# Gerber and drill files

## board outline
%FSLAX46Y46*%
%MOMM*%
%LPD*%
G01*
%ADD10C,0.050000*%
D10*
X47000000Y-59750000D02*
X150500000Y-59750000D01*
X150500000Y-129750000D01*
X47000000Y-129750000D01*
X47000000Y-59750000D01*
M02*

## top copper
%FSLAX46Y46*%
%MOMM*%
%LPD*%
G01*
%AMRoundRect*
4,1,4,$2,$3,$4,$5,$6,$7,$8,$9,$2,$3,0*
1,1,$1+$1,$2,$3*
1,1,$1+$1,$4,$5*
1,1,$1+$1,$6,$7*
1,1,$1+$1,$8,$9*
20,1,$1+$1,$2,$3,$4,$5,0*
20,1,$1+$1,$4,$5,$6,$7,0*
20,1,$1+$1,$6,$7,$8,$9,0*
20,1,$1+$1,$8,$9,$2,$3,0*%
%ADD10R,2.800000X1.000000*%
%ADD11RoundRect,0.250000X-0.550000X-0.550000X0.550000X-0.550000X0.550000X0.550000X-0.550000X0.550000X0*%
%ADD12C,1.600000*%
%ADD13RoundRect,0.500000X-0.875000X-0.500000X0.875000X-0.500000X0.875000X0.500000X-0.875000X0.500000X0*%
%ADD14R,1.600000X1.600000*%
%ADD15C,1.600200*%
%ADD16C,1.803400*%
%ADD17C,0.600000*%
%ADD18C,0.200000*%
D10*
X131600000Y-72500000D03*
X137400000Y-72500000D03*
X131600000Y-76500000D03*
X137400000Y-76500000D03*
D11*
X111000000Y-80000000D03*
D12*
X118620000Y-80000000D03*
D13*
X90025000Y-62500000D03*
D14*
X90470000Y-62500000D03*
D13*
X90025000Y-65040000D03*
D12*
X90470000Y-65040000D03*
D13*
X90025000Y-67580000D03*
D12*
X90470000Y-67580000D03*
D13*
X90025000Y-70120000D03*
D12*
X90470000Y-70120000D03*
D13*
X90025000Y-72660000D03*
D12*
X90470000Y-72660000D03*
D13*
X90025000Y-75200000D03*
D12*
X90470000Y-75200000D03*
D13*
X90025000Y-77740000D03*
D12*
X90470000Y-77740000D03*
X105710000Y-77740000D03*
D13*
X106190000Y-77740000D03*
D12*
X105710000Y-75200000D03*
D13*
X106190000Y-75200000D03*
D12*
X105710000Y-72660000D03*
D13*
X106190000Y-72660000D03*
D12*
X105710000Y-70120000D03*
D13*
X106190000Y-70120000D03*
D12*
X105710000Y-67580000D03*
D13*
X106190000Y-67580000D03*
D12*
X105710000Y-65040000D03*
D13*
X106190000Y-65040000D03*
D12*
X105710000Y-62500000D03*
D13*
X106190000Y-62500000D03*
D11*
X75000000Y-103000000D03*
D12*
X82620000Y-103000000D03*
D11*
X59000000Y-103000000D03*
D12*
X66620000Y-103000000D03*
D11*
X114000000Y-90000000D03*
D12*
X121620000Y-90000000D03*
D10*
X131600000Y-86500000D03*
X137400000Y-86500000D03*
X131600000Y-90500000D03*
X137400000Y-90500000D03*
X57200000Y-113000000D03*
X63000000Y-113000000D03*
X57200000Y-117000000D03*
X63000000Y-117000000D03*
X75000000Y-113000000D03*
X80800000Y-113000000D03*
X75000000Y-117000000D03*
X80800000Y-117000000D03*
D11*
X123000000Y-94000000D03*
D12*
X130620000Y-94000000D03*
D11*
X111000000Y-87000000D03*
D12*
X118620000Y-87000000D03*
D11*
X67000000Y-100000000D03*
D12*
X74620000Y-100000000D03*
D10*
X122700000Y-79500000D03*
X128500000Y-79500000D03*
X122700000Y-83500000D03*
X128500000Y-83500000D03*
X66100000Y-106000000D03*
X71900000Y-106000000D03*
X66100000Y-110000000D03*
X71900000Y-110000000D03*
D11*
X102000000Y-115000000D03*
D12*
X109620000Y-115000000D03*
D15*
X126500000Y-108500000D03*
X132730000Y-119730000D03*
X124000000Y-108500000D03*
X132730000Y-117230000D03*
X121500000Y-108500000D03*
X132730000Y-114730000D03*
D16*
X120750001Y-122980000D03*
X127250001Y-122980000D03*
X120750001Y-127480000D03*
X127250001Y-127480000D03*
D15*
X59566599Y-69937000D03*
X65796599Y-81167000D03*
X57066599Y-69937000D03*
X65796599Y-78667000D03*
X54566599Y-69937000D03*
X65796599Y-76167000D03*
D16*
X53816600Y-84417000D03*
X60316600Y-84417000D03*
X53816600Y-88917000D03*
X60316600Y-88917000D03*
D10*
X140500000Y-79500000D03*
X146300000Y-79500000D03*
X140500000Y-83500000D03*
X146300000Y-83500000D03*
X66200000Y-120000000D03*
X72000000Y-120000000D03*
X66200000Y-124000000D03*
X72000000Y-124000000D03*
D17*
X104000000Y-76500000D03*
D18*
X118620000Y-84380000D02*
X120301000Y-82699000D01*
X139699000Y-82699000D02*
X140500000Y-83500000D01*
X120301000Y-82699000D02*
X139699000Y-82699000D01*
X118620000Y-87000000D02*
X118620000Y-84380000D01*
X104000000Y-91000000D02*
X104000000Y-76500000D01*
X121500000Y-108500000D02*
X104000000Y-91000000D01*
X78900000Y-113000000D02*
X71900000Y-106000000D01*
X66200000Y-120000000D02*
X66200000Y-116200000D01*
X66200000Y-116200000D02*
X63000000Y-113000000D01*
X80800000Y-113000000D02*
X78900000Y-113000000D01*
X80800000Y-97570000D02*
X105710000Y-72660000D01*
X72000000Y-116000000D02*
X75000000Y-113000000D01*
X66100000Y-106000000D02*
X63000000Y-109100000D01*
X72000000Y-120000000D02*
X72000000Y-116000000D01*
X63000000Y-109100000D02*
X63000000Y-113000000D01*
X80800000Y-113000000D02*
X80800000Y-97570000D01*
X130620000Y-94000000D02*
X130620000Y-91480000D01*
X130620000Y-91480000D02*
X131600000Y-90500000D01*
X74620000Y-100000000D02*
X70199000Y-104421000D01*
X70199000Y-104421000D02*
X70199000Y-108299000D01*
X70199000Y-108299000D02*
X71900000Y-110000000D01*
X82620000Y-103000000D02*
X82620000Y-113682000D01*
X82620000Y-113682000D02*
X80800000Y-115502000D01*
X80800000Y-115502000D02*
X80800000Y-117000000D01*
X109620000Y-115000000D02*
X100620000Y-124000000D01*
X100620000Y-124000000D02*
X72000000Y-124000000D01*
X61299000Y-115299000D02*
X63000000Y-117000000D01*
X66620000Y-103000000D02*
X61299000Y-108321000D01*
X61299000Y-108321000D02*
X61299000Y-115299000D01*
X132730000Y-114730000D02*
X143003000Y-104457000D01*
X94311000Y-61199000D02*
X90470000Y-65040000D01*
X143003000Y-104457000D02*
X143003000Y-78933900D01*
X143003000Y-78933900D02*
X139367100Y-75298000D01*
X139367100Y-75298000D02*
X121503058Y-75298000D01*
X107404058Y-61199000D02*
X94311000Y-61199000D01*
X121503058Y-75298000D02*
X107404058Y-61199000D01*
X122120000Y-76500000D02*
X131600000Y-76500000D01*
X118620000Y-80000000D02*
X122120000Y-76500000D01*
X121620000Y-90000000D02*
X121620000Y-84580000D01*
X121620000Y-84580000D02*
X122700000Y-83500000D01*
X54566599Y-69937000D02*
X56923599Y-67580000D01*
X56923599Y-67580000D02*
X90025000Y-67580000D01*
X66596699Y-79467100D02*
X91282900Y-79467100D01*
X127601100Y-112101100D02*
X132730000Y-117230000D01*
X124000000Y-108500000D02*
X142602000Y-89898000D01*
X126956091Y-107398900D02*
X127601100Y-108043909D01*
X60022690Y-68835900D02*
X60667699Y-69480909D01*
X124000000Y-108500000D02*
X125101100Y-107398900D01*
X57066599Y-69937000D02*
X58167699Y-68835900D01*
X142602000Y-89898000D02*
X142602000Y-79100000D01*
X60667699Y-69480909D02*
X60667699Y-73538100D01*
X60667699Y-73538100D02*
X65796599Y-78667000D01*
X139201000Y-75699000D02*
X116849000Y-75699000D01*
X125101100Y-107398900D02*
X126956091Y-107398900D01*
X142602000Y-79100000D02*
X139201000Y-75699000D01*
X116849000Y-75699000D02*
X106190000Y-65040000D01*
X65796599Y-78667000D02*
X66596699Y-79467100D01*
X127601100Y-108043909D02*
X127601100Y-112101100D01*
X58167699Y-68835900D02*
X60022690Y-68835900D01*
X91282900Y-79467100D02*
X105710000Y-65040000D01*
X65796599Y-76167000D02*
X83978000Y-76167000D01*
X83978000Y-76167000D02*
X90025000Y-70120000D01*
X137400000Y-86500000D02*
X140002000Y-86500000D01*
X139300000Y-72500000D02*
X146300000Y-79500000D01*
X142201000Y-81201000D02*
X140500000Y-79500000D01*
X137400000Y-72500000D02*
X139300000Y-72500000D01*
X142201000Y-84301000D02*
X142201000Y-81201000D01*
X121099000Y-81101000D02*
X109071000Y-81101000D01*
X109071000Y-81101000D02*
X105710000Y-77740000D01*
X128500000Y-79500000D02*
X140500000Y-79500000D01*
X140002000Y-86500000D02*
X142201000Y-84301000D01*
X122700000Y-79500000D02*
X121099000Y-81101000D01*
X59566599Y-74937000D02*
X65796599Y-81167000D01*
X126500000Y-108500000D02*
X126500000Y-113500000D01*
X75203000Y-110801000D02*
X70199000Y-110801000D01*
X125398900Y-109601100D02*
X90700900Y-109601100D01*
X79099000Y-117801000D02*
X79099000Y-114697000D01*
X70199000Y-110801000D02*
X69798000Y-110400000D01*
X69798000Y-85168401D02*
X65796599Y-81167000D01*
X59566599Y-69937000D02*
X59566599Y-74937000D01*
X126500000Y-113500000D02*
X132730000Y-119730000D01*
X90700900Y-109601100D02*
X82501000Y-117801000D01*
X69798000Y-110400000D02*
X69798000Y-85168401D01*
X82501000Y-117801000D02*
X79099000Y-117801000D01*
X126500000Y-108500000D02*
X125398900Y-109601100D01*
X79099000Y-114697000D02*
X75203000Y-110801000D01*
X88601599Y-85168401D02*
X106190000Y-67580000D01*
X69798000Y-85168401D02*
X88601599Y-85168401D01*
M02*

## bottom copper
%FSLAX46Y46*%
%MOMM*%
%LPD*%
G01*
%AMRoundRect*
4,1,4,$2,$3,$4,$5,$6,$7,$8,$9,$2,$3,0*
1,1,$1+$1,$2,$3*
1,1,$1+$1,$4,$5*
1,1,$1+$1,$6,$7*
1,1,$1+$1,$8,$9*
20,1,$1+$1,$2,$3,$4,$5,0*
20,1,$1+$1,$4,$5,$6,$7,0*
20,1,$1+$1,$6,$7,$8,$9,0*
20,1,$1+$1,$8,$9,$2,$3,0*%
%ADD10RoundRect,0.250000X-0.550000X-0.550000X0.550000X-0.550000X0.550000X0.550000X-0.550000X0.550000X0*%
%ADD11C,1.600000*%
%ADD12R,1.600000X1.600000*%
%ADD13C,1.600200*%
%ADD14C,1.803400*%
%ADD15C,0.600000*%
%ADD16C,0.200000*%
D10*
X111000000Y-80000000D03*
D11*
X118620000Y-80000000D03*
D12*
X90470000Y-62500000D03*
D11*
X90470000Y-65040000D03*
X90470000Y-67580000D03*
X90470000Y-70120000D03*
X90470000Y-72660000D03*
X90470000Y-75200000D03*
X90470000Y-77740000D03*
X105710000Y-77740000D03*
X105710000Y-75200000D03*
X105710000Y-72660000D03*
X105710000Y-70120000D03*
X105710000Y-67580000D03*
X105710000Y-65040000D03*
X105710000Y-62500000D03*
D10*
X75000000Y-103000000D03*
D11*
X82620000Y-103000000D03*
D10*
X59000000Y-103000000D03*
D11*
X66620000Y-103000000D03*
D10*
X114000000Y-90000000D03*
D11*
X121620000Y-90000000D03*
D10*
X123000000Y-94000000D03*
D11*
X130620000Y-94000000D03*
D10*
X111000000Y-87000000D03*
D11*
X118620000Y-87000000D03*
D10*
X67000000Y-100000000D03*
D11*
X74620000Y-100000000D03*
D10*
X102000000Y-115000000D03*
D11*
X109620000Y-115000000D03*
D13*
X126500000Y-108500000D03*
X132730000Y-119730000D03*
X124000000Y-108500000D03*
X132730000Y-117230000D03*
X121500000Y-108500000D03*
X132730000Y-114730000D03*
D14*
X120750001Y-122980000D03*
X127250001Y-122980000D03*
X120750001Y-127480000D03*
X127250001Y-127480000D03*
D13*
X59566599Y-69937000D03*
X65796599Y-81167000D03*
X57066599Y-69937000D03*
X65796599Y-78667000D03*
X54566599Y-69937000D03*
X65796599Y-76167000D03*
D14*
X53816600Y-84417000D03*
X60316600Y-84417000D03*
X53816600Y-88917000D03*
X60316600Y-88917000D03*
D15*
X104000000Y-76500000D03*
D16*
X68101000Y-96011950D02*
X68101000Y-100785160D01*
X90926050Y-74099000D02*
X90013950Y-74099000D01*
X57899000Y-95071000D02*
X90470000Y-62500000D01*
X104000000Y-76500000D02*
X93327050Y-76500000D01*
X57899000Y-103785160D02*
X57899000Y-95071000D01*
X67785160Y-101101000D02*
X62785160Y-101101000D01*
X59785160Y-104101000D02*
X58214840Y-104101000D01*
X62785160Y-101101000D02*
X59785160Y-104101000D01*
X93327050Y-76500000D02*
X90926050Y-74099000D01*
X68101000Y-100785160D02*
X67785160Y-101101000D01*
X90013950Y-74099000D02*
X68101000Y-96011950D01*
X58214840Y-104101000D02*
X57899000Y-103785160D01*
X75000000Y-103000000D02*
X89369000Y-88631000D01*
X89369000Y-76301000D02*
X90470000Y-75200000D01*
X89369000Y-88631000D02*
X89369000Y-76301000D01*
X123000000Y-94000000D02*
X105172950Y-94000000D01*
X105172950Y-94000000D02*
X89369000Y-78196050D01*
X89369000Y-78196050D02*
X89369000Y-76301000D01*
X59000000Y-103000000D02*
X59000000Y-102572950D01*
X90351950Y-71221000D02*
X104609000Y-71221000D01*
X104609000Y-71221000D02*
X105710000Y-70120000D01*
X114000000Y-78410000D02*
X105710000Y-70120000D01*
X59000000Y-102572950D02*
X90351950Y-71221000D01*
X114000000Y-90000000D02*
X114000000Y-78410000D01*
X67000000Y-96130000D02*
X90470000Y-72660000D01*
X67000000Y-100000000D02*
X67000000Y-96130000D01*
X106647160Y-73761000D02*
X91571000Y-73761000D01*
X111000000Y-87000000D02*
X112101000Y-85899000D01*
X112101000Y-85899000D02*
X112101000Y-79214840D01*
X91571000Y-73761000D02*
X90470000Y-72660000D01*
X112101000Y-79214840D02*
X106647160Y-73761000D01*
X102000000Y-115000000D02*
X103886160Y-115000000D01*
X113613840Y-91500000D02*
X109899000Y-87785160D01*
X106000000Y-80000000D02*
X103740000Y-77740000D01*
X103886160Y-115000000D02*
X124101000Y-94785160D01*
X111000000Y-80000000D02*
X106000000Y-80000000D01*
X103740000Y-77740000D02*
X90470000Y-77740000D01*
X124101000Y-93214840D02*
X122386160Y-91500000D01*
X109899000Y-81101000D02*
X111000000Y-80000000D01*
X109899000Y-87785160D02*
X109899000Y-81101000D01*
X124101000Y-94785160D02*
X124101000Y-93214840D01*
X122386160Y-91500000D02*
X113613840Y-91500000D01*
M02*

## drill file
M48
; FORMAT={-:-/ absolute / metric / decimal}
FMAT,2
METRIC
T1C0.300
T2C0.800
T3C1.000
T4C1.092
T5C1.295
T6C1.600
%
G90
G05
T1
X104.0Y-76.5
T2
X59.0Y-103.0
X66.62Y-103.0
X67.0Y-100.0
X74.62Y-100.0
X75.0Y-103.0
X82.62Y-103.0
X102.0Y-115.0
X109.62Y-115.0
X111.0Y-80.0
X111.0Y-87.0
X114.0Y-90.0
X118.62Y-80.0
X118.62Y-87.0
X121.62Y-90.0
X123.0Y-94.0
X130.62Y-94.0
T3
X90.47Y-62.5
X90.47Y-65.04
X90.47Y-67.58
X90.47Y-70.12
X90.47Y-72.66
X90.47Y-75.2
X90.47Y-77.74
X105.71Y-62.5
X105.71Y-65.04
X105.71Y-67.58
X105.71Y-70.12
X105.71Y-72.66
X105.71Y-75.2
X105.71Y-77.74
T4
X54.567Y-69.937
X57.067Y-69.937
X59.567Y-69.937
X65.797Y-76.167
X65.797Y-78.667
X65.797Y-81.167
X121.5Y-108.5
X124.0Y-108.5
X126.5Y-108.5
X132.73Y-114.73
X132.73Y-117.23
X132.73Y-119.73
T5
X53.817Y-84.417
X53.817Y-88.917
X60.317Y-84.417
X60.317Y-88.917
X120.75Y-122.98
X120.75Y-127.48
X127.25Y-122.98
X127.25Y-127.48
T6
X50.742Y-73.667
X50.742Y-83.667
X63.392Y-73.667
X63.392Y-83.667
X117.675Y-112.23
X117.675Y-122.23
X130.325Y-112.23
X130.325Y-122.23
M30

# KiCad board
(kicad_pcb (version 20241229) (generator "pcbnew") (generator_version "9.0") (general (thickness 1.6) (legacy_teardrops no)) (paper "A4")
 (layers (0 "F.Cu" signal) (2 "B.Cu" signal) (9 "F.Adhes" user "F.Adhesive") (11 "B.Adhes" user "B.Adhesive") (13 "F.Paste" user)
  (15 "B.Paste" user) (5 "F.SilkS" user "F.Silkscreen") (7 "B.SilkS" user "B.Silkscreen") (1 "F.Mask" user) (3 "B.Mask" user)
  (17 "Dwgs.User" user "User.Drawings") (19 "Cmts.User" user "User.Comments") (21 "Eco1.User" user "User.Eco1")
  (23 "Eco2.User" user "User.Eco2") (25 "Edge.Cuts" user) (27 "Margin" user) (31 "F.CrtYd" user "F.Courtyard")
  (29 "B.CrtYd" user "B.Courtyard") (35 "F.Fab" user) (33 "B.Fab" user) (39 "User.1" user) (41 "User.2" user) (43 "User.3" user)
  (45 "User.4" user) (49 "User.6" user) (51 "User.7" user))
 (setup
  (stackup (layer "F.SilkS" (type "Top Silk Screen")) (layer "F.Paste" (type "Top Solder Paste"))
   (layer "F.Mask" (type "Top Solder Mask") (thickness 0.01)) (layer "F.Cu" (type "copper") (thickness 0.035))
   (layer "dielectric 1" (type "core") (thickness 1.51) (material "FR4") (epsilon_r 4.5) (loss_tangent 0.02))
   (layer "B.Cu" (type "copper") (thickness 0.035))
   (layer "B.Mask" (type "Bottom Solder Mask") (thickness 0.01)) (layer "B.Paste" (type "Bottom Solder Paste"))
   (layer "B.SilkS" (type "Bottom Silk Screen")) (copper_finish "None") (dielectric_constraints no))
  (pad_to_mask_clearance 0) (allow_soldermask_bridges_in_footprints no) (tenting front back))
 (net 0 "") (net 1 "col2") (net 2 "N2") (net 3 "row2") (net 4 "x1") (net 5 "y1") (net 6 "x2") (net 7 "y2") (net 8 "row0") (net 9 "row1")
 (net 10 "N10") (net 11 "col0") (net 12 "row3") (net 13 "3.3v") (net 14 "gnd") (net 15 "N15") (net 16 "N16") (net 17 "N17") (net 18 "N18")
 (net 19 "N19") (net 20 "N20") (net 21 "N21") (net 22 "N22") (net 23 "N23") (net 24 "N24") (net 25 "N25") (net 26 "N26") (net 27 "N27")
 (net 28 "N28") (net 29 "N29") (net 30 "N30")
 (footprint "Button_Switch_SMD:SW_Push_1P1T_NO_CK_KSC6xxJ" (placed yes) (layer "F.Cu") (at 134.5 74.5)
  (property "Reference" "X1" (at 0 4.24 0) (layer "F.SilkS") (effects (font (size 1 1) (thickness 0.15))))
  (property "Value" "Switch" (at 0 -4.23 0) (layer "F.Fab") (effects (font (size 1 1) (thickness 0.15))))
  (pad "1" smd rect (at -2.9 -2) (size 2.8 1) (layers "F.Cu" "F.Mask" "F.Paste") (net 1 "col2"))
  (pad "1" smd rect (at 2.9 -2) (size 2.8 1) (layers "F.Cu" "F.Mask" "F.Paste") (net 1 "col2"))
  (pad "2" smd rect (at -2.9 2) (size 2.8 1) (layers "F.Cu" "F.Mask" "F.Paste") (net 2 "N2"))
  (pad "2" smd rect (at 2.9 2) (size 2.8 1) (layers "F.Cu" "F.Mask" "F.Paste") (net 2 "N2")))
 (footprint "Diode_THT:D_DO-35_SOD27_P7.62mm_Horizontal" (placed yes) (layer "F.Cu") (at 111 80)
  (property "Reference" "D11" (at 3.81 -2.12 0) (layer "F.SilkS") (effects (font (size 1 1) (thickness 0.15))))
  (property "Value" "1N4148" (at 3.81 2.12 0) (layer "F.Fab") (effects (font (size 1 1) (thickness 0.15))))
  (pad "1" thru_hole roundrect (at 0 0) (size 1.6 1.6) (drill 0.8) (layers "*.Cu" "*.Mask") (remove_unused_layers no)
   (roundrect_rratio 0.15625) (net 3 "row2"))
  (pad "2" thru_hole circle (at 7.62 0) (size 1.6 1.6) (drill 0.8) (layers "*.Cu" "*.Mask") (remove_unused_layers no) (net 2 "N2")))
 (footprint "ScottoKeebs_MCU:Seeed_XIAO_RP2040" (layer "F.Cu") (at 98.09 70.12)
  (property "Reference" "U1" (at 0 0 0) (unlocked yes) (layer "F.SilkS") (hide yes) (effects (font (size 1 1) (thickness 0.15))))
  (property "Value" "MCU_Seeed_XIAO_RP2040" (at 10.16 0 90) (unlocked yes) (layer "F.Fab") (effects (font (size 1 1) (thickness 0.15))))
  (pad "1" smd roundrect (at -8.065 -7.62) (size 2.75 2) (layers "F.Cu" "F.Mask" "F.Paste") (roundrect_rratio 0.25) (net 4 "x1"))
  (pad "1" thru_hole rect (at -7.62 -7.62 90) (size 1.6 1.6) (drill 1) (layers "*.Cu" "*.Mask") (remove_unused_layers no) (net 4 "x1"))
  (pad "2" smd roundrect (at -8.065 -5.08) (size 2.75 2) (layers "F.Cu" "F.Mask" "F.Paste") (roundrect_rratio 0.25) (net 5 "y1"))
  (pad "2" thru_hole circle (at -7.62 -5.08 90) (size 1.6 1.6) (drill 1) (layers "*.Cu" "*.Mask") (remove_unused_layers no) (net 5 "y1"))
  (pad "3" smd roundrect (at -8.065 -2.54) (size 2.75 2) (layers "F.Cu" "F.Mask" "F.Paste") (roundrect_rratio 0.25) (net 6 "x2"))
  (pad "3" thru_hole circle (at -7.62 -2.54 90) (size 1.6 1.6) (drill 1) (layers "*.Cu" "*.Mask") (remove_unused_layers no) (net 6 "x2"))
  (pad "4" smd roundrect (at -8.065 0) (size 2.75 2) (layers "F.Cu" "F.Mask" "F.Paste") (roundrect_rratio 0.25) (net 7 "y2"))
  (pad "4" thru_hole circle (at -7.62 0 90) (size 1.6 1.6) (drill 1) (layers "*.Cu" "*.Mask") (remove_unused_layers no) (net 7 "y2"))
  (pad "5" smd roundrect (at -8.065 2.54) (size 2.75 2) (layers "F.Cu" "F.Mask" "F.Paste") (roundrect_rratio 0.25) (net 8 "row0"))
  (pad "5" thru_hole circle (at -7.62 2.54 90) (size 1.6 1.6) (drill 1) (layers "*.Cu" "*.Mask") (remove_unused_layers no) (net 8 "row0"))
  (pad "6" smd roundrect (at -8.065 5.08) (size 2.75 2) (layers "F.Cu" "F.Mask" "F.Paste") (roundrect_rratio 0.25) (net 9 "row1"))
  (pad "6" thru_hole circle (at -7.62 5.08 90) (size 1.6 1.6) (drill 1) (layers "*.Cu" "*.Mask") (remove_unused_layers no) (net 9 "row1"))
  (pad "7" smd roundrect (at -8.065 7.62) (size 2.75 2) (layers "F.Cu" "F.Mask" "F.Paste") (roundrect_rratio 0.25) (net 3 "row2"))
  (pad "7" thru_hole circle (at -7.62 7.62 90) (size 1.6 1.6) (drill 1) (layers "*.Cu" "*.Mask") (remove_unused_layers no) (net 3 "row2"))
  (pad "8" thru_hole circle (at 7.62 7.62 90) (size 1.6 1.6) (drill 1) (layers "*.Cu" "*.Mask") (remove_unused_layers no) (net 1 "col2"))
  (pad "8" smd roundrect (at 8.1 7.62) (size 2.75 2) (layers "F.Cu" "F.Mask" "F.Paste") (roundrect_rratio 0.25) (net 1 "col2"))
  (pad "9" thru_hole circle (at 7.62 5.08 90) (size 1.6 1.6) (drill 1) (layers "*.Cu" "*.Mask") (remove_unused_layers no) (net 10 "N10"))
  (pad "9" smd roundrect (at 8.1 5.08) (size 2.75 2) (layers "F.Cu" "F.Mask" "F.Paste") (roundrect_rratio 0.25) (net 10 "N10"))
  (pad "10" thru_hole circle (at 7.62 2.54 90) (size 1.6 1.6) (drill 1) (layers "*.Cu" "*.Mask") (remove_unused_layers no) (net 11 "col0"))
  (pad "10" smd roundrect (at 8.1 2.54) (size 2.75 2) (layers "F.Cu" "F.Mask" "F.Paste") (roundrect_rratio 0.25) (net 11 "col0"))
  (pad "11" thru_hole circle (at 7.62 0 90) (size 1.6 1.6) (drill 1) (layers "*.Cu" "*.Mask") (remove_unused_layers no) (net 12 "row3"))
  (pad "11" smd roundrect (at 8.1 0) (size 2.75 2) (layers "F.Cu" "F.Mask" "F.Paste") (roundrect_rratio 0.25) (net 12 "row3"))
  (pad "12" thru_hole circle (at 7.62 -2.54 90) (size 1.6 1.6) (drill 1) (layers "*.Cu" "*.Mask") (remove_unused_layers no) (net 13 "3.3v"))
  (pad "12" smd roundrect (at 8.1 -2.54) (size 2.75 2) (layers "F.Cu" "F.Mask" "F.Paste") (roundrect_rratio 0.25) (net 13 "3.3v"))
  (pad "13" thru_hole circle (at 7.62 -5.08 90) (size 1.6 1.6) (drill 1) (layers "*.Cu" "*.Mask") (remove_unused_layers no) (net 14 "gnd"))
  (pad "13" smd roundrect (at 8.1 -5.08) (size 2.75 2) (layers "F.Cu" "F.Mask" "F.Paste") (roundrect_rratio 0.25) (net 14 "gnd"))
  (pad "14" thru_hole circle (at 7.62 -7.62 90) (size 1.6 1.6) (drill 1) (layers "*.Cu" "*.Mask") (remove_unused_layers no) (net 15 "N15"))
  (pad "14" smd roundrect (at 8.1 -7.62) (size 2.75 2) (layers "F.Cu" "F.Mask" "F.Paste") (roundrect_rratio 0.25) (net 15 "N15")))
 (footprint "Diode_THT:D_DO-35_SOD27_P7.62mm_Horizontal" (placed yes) (layer "F.Cu") (at 75 103)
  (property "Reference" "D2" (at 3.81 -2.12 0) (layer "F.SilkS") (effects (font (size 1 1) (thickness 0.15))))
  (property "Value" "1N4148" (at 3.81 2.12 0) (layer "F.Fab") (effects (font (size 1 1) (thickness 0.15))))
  (pad "1" thru_hole roundrect (at 0 0) (size 1.6 1.6) (drill 0.8) (layers "*.Cu" "*.Mask") (remove_unused_layers no)
   (roundrect_rratio 0.15625) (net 9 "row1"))
  (pad "2" thru_hole circle (at 7.62 0) (size 1.6 1.6) (drill 0.8) (layers "*.Cu" "*.Mask") (remove_unused_layers no) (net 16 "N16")))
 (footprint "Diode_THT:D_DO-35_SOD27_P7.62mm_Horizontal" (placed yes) (layer "F.Cu") (at 59 103)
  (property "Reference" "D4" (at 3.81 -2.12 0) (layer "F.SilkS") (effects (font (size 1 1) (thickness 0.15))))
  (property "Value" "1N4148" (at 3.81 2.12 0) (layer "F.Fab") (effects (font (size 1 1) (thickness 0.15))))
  (pad "1" thru_hole roundrect (at 0 0) (size 1.6 1.6) (drill 0.8) (layers "*.Cu" "*.Mask") (remove_unused_layers no)
   (roundrect_rratio 0.15625) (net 12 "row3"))
  (pad "2" thru_hole circle (at 7.62 0) (size 1.6 1.6) (drill 0.8) (layers "*.Cu" "*.Mask") (remove_unused_layers no) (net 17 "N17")))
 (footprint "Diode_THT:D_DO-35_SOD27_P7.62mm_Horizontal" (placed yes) (layer "F.Cu") (at 114 90)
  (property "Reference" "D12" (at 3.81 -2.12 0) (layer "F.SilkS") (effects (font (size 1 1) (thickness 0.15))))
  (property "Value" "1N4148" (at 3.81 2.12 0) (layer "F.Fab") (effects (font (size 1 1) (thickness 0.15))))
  (pad "1" thru_hole roundrect (at 0 0) (size 1.6 1.6) (drill 0.8) (layers "*.Cu" "*.Mask") (remove_unused_layers no)
   (roundrect_rratio 0.15625) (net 12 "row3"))
  (pad "2" thru_hole circle (at 7.62 0) (size 1.6 1.6) (drill 0.8) (layers "*.Cu" "*.Mask") (remove_unused_layers no) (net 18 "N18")))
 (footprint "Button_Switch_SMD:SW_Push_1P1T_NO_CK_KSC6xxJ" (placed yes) (layer "F.Cu") (at 134.5 88.5)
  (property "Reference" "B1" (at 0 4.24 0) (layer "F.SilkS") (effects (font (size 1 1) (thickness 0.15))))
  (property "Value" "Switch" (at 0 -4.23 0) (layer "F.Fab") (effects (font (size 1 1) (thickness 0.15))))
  (pad "1" smd rect (at -2.9 -2) (size 2.8 1) (layers "F.Cu" "F.Mask" "F.Paste") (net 1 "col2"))
  (pad "1" smd rect (at 2.9 -2) (size 2.8 1) (layers "F.Cu" "F.Mask" "F.Paste") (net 1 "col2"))
  (pad "2" smd rect (at -2.9 2) (size 2.8 1) (layers "F.Cu" "F.Mask" "F.Paste") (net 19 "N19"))
  (pad "2" smd rect (at 2.9 2) (size 2.8 1) (layers "F.Cu" "F.Mask" "F.Paste") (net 19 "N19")))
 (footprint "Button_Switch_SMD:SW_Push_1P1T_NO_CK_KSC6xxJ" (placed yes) (layer "F.Cu") (at 60.1 115)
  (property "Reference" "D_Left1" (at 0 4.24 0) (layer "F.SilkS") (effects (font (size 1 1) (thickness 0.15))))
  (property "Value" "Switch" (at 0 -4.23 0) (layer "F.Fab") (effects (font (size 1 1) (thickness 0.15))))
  (pad "1" smd rect (at -2.9 -2) (size 2.8 1) (layers "F.Cu" "F.Mask" "F.Paste") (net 11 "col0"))
  (pad "1" smd rect (at 2.9 -2) (size 2.8 1) (layers "F.Cu" "F.Mask" "F.Paste") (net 11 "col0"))
  (pad "2" smd rect (at -2.9 2) (size 2.8 1) (layers "F.Cu" "F.Mask" "F.Paste") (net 17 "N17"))
  (pad "2" smd rect (at 2.9 2) (size 2.8 1) (layers "F.Cu" "F.Mask" "F.Paste") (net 17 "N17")))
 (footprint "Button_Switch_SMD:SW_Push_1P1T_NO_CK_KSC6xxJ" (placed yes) (layer "F.Cu") (at 77.9 115)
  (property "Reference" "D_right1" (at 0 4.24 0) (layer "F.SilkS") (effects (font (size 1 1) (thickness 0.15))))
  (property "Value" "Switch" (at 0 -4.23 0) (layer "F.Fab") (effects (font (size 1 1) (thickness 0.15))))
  (pad "1" smd rect (at -2.9 -2) (size 2.8 1) (layers "F.Cu" "F.Mask" "F.Paste") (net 11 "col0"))
  (pad "1" smd rect (at 2.9 -2) (size 2.8 1) (layers "F.Cu" "F.Mask" "F.Paste") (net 11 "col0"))
  (pad "2" smd rect (at -2.9 2) (size 2.8 1) (layers "F.Cu" "F.Mask" "F.Paste") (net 16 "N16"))
  (pad "2" smd rect (at 2.9 2) (size 2.8 1) (layers "F.Cu" "F.Mask" "F.Paste") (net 16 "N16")))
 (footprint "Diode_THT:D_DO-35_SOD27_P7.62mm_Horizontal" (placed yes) (layer "F.Cu") (at 123 94)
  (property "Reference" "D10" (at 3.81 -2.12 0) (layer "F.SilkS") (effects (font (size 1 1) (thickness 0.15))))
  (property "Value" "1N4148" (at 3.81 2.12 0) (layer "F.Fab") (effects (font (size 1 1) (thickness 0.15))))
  (pad "1" thru_hole roundrect (at 0 0) (size 1.6 1.6) (drill 0.8) (layers "*.Cu" "*.Mask") (remove_unused_layers no)
   (roundrect_rratio 0.15625) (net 9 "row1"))
  (pad "2" thru_hole circle (at 7.62 0) (size 1.6 1.6) (drill 0.8) (layers "*.Cu" "*.Mask") (remove_unused_layers no) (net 19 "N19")))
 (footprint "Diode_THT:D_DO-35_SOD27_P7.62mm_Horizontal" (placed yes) (layer "F.Cu") (at 111 87)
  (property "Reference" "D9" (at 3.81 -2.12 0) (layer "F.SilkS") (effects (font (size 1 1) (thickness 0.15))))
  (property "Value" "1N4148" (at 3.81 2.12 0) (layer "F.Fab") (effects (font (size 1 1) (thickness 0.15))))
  (pad "1" thru_hole roundrect (at 0 0) (size 1.6 1.6) (drill 0.8) (layers "*.Cu" "*.Mask") (remove_unused_layers no)
   (roundrect_rratio 0.15625) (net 8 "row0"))
  (pad "2" thru_hole circle (at 7.62 0) (size 1.6 1.6) (drill 0.8) (layers "*.Cu" "*.Mask") (remove_unused_layers no) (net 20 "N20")))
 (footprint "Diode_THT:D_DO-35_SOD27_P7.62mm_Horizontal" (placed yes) (layer "F.Cu") (at 67 100)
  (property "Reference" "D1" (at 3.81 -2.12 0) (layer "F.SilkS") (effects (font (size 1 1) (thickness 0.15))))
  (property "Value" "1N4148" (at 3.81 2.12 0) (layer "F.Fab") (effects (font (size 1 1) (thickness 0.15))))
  (pad "1" thru_hole roundrect (at 0 0) (size 1.6 1.6) (drill 0.8) (layers "*.Cu" "*.Mask") (remove_unused_layers no)
   (roundrect_rratio 0.15625) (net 8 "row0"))
  (pad "2" thru_hole circle (at 7.62 0) (size 1.6 1.6) (drill 0.8) (layers "*.Cu" "*.Mask") (remove_unused_layers no) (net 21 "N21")))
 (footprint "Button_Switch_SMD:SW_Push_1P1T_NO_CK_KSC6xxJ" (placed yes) (layer "F.Cu") (at 125.6 81.5)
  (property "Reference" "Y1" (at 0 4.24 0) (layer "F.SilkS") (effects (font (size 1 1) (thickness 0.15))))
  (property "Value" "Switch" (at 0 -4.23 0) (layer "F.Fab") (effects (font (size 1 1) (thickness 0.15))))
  (pad "1" smd rect (at -2.9 -2) (size 2.8 1) (layers "F.Cu" "F.Mask" "F.Paste") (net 1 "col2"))
  (pad "1" smd rect (at 2.9 -2) (size 2.8 1) (layers "F.Cu" "F.Mask" "F.Paste") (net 1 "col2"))
  (pad "2" smd rect (at -2.9 2) (size 2.8 1) (layers "F.Cu" "F.Mask" "F.Paste") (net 18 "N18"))
  (pad "2" smd rect (at 2.9 2) (size 2.8 1) (layers "F.Cu" "F.Mask" "F.Paste") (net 18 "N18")))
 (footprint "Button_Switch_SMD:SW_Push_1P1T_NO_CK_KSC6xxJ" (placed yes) (layer "F.Cu") (at 69 108)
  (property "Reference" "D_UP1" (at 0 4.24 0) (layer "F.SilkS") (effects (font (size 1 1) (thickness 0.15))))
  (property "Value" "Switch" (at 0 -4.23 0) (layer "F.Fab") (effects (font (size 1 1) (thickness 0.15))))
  (pad "1" smd rect (at -2.9 -2) (size 2.8 1) (layers "F.Cu" "F.Mask" "F.Paste") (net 11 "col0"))
  (pad "1" smd rect (at 2.9 -2) (size 2.8 1) (layers "F.Cu" "F.Mask" "F.Paste") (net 11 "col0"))
  (pad "2" smd rect (at -2.9 2) (size 2.8 1) (layers "F.Cu" "F.Mask" "F.Paste") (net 21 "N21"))
  (pad "2" smd rect (at 2.9 2) (size 2.8 1) (layers "F.Cu" "F.Mask" "F.Paste") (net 21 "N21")))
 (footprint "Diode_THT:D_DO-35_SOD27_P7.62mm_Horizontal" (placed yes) (layer "F.Cu") (at 102 115)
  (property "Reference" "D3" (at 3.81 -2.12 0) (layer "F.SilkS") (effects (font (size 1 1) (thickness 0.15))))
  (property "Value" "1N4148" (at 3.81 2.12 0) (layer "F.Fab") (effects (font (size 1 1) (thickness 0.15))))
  (pad "1" thru_hole roundrect (at 0 0) (size 1.6 1.6) (drill 0.8) (layers "*.Cu" "*.Mask") (remove_unused_layers no)
   (roundrect_rratio 0.15625) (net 3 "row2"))
  (pad "2" thru_hole circle (at 7.62 0) (size 1.6 1.6) (drill 0.8) (layers "*.Cu" "*.Mask") (remove_unused_layers no) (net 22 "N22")))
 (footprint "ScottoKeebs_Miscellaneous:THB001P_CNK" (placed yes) (layer "F.Cu") (at 126.5 108.5)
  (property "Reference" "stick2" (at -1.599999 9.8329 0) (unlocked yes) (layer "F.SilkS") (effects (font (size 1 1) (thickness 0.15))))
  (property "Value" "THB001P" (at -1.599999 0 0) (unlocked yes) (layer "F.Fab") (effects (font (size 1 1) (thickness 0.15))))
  (pad "" np_thru_hole circle (at -8.824999 3.73) (size 1.6002 1.6002) (drill 1.6002) (layers))
  (pad "" np_thru_hole circle (at -8.824999 13.73) (size 1.6002 1.6002) (drill 1.6002) (layers))
  (pad "" np_thru_hole circle (at 3.825001 3.73) (size 1.6002 1.6002) (drill 1.6002) (layers))
  (pad "" np_thru_hole circle (at 3.825001 13.73) (size 1.6002 1.6002) (drill 1.6002) (layers))
  (pad "1" thru_hole circle (at 0 0) (size 1.6002 1.6002) (drill 1.0922) (layers "*.Cu" "*.Mask") (remove_unused_layers no) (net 13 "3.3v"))
  (pad "1'" thru_hole circle (at 6.23 11.23) (size 1.6002 1.6002) (drill 1.0922) (layers "*.Cu" "*.Mask") (remove_unused_layers no)
   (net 13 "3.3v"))
  (pad "2" thru_hole circle (at -2.5 0) (size 1.6002 1.6002) (drill 1.0922) (layers "*.Cu" "*.Mask") (remove_unused_layers no)
   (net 14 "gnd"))
  (pad "2'" thru_hole circle (at 6.23 8.73) (size 1.6002 1.6002) (drill 1.0922) (layers "*.Cu" "*.Mask") (remove_unused_layers no)
   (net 14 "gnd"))
  (pad "3" thru_hole circle (at -5 0) (size 1.6002 1.6002) (drill 1.0922) (layers "*.Cu" "*.Mask") (remove_unused_layers no) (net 4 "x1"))
  (pad "3'" thru_hole circle (at 6.23 6.23) (size 1.6002 1.6002) (drill 1.0922) (layers "*.Cu" "*.Mask") (remove_unused_layers no)
   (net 5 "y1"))
  (pad "A" thru_hole circle (at -5.749999 14.48) (size 1.8034 1.8034) (drill 1.2954) (layers "*.Cu" "*.Mask") (remove_unused_layers no)
   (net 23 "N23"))
  (pad "B" thru_hole circle (at 0.750001 14.48) (size 1.8034 1.8034) (drill 1.2954) (layers "*.Cu" "*.Mask") (remove_unused_layers no)
   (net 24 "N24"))
  (pad "C" thru_hole circle (at -5.749999 18.98) (size 1.8034 1.8034) (drill 1.2954) (layers "*.Cu" "*.Mask") (remove_unused_layers no)
   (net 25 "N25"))
  (pad "D" thru_hole circle (at 0.750001 18.98) (size 1.8034 1.8034) (drill 1.2954) (layers "*.Cu" "*.Mask") (remove_unused_layers no)
   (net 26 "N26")))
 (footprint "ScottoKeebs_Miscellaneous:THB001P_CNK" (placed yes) (layer "F.Cu") (at 59.566599 69.937)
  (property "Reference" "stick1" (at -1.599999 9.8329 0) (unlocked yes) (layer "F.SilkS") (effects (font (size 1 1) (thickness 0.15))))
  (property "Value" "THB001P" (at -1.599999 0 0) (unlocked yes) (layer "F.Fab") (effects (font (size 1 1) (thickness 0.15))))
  (pad "" np_thru_hole circle (at -8.824999 3.73) (size 1.6002 1.6002) (drill 1.6002) (layers))
  (pad "" np_thru_hole circle (at -8.824999 13.73) (size 1.6002 1.6002) (drill 1.6002) (layers))
  (pad "" np_thru_hole circle (at 3.825001 3.73) (size 1.6002 1.6002) (drill 1.6002) (layers))
  (pad "" np_thru_hole circle (at 3.825001 13.73) (size 1.6002 1.6002) (drill 1.6002) (layers))
  (pad "1" thru_hole circle (at 0 0) (size 1.6002 1.6002) (drill 1.0922) (layers "*.Cu" "*.Mask") (remove_unused_layers no) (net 13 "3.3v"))
  (pad "1'" thru_hole circle (at 6.23 11.23) (size 1.6002 1.6002) (drill 1.0922) (layers "*.Cu" "*.Mask") (remove_unused_layers no)
   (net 13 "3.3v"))
  (pad "2" thru_hole circle (at -2.5 0) (size 1.6002 1.6002) (drill 1.0922) (layers "*.Cu" "*.Mask") (remove_unused_layers no)
   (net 14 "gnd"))
  (pad "2'" thru_hole circle (at 6.23 8.73) (size 1.6002 1.6002) (drill 1.0922) (layers "*.Cu" "*.Mask") (remove_unused_layers no)
   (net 14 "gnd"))
  (pad "3" thru_hole circle (at -5 0) (size 1.6002 1.6002) (drill 1.0922) (layers "*.Cu" "*.Mask") (remove_unused_layers no) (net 6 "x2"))
  (pad "3'" thru_hole circle (at 6.23 6.23) (size 1.6002 1.6002) (drill 1.0922) (layers "*.Cu" "*.Mask") (remove_unused_layers no)
   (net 7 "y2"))
  (pad "A" thru_hole circle (at -5.749999 14.48) (size 1.8034 1.8034) (drill 1.2954) (layers "*.Cu" "*.Mask") (remove_unused_layers no)
   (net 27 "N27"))
  (pad "B" thru_hole circle (at 0.750001 14.48) (size 1.8034 1.8034) (drill 1.2954) (layers "*.Cu" "*.Mask") (remove_unused_layers no)
   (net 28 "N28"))
  (pad "C" thru_hole circle (at -5.749999 18.98) (size 1.8034 1.8034) (drill 1.2954) (layers "*.Cu" "*.Mask") (remove_unused_layers no)
   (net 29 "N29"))
  (pad "D" thru_hole circle (at 0.750001 18.98) (size 1.8034 1.8034) (drill 1.2954) (layers "*.Cu" "*.Mask") (remove_unused_layers no)
   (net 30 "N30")))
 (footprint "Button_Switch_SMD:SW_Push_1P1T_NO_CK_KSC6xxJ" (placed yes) (layer "F.Cu") (at 143.4 81.5)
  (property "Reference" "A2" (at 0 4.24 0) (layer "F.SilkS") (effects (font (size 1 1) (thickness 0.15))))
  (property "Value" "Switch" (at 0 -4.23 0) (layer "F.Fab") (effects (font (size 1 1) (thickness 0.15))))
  (pad "1" smd rect (at -2.9 -2) (size 2.8 1) (layers "F.Cu" "F.Mask" "F.Paste") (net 1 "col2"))
  (pad "1" smd rect (at 2.9 -2) (size 2.8 1) (layers "F.Cu" "F.Mask" "F.Paste") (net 1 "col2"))
  (pad "2" smd rect (at -2.9 2) (size 2.8 1) (layers "F.Cu" "F.Mask" "F.Paste") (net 20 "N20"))
  (pad "2" smd rect (at 2.9 2) (size 2.8 1) (layers "F.Cu" "F.Mask" "F.Paste") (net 20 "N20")))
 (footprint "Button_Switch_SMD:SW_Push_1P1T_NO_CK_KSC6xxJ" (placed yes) (layer "F.Cu") (at 69.1 122)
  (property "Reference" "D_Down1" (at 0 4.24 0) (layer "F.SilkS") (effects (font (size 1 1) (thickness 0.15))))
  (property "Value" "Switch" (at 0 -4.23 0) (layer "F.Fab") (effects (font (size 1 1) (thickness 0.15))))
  (pad "1" smd rect (at -2.9 -2) (size 2.8 1) (layers "F.Cu" "F.Mask" "F.Paste") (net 11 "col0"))
  (pad "1" smd rect (at 2.9 -2) (size 2.8 1) (layers "F.Cu" "F.Mask" "F.Paste") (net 11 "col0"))
  (pad "2" smd rect (at -2.9 2) (size 2.8 1) (layers "F.Cu" "F.Mask" "F.Paste") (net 22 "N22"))
  (pad "2" smd rect (at 2.9 2) (size 2.8 1) (layers "F.Cu" "F.Mask" "F.Paste") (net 22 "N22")))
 (gr_rect (start 47 59.75) (end 150.5 129.75) (stroke (width 0.05) (type solid)) (fill no) (layer "Edge.Cuts"))
 (segment (start 118.62 84.38) (end 120.301 82.699) (width 0.2) (layer "F.Cu") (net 20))
 (segment (start 139.699 82.699) (end 140.5 83.5) (width 0.2) (layer "F.Cu") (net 20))
 (segment (start 120.301 82.699) (end 139.699 82.699) (width 0.2) (layer "F.Cu") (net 20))
 (segment (start 118.62 87) (end 118.62 84.38) (width 0.2) (layer "F.Cu") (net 20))
 (segment (start 104 91) (end 104 76.5) (width 0.2) (layer "F.Cu") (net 4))
 (segment (start 121.5 108.5) (end 104 91) (width 0.2) (layer "F.Cu") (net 4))
 (via (at 104 76.5) (size 0.6) (drill 0.3) (layers "F.Cu" "B.Cu") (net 4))
 (segment (start 68.101 96.01195) (end 68.101 100.78516) (width 0.2) (layer "B.Cu") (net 4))
 (segment (start 90.92605 74.099) (end 90.01395 74.099) (width 0.2) (layer "B.Cu") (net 4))
 (segment (start 57.899 95.071) (end 90.47 62.5) (width 0.2) (layer "B.Cu") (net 4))
 (segment (start 104 76.5) (end 93.32705 76.5) (width 0.2) (layer "B.Cu") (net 4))
 (segment (start 57.899 103.78516) (end 57.899 95.071) (width 0.2) (layer "B.Cu") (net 4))
 (segment (start 67.78516 101.101) (end 62.78516 101.101) (width 0.2) (layer "B.Cu") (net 4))
 (segment (start 59.78516 104.101) (end 58.21484 104.101) (width 0.2) (layer "B.Cu") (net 4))
 (segment (start 62.78516 101.101) (end 59.78516 104.101) (width 0.2) (layer "B.Cu") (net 4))
 (segment (start 93.32705 76.5) (end 90.92605 74.099) (width 0.2) (layer "B.Cu") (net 4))
 (segment (start 68.101 100.78516) (end 67.78516 101.101) (width 0.2) (layer "B.Cu") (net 4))
 (segment (start 90.01395 74.099) (end 68.101 96.01195) (width 0.2) (layer "B.Cu") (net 4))
 (segment (start 58.21484 104.101) (end 57.899 103.78516) (width 0.2) (layer "B.Cu") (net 4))
 (segment (start 78.9 113) (end 71.9 106) (width 0.2) (layer "F.Cu") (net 11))
 (segment (start 66.2 120) (end 66.2 116.2) (width 0.2) (layer "F.Cu") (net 11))
 (segment (start 66.2 116.2) (end 63 113) (width 0.2) (layer "F.Cu") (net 11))
 (segment (start 80.8 113) (end 78.9 113) (width 0.2) (layer "F.Cu") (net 11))
 (segment (start 80.8 97.57) (end 105.71 72.66) (width 0.2) (layer "F.Cu") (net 11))
 (segment (start 72 116) (end 75 113) (width 0.2) (layer "F.Cu") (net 11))
 (segment (start 66.1 106) (end 63 109.1) (width 0.2) (layer "F.Cu") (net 11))
 (segment (start 72 120) (end 72 116) (width 0.2) (layer "F.Cu") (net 11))
 (segment (start 63 109.1) (end 63 113) (width 0.2) (layer "F.Cu") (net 11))
 (segment (start 80.8 113) (end 80.8 97.57) (width 0.2) (layer "F.Cu") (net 11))
 (segment (start 130.62 94) (end 130.62 91.48) (width 0.2) (layer "F.Cu") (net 19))
 (segment (start 130.62 91.48) (end 131.6 90.5) (width 0.2) (layer "F.Cu") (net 19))
 (segment (start 74.62 100) (end 70.199 104.421) (width 0.2) (layer "F.Cu") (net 21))
 (segment (start 70.199 104.421) (end 70.199 108.299) (width 0.2) (layer "F.Cu") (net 21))
 (segment (start 70.199 108.299) (end 71.9 110) (width 0.2) (layer "F.Cu") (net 21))
 (segment (start 82.62 103) (end 82.62 113.682) (width 0.2) (layer "F.Cu") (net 16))
 (segment (start 82.62 113.682) (end 80.8 115.502) (width 0.2) (layer "F.Cu") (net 16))
 (segment (start 80.8 115.502) (end 80.8 117) (width 0.2) (layer "F.Cu") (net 16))
 (segment (start 109.62 115) (end 100.62 124) (width 0.2) (layer "F.Cu") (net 22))
 (segment (start 100.62 124) (end 72 124) (width 0.2) (layer "F.Cu") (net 22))
 (segment (start 61.299 115.299) (end 63 117) (width 0.2) (layer "F.Cu") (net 17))
 (segment (start 66.62 103) (end 61.299 108.321) (width 0.2) (layer "F.Cu") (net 17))
 (segment (start 61.299 108.321) (end 61.299 115.299) (width 0.2) (layer "F.Cu") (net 17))
 (segment (start 132.73 114.73) (end 143.003 104.457) (width 0.2) (layer "F.Cu") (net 5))
 (segment (start 94.311 61.199) (end 90.47 65.04) (width 0.2) (layer "F.Cu") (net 5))
 (segment (start 143.003 104.457) (end 143.003 78.9339) (width 0.2) (layer "F.Cu") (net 5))
 (segment (start 143.003 78.9339) (end 139.3671 75.298) (width 0.2) (layer "F.Cu") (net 5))
 (segment (start 139.3671 75.298) (end 121.503058 75.298) (width 0.2) (layer "F.Cu") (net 5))
 (segment (start 107.404058 61.199) (end 94.311 61.199) (width 0.2) (layer "F.Cu") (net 5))
 (segment (start 121.503058 75.298) (end 107.404058 61.199) (width 0.2) (layer "F.Cu") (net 5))
 (segment (start 122.12 76.5) (end 131.6 76.5) (width 0.2) (layer "F.Cu") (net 2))
 (segment (start 118.62 80) (end 122.12 76.5) (width 0.2) (layer "F.Cu") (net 2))
 (segment (start 121.62 90) (end 121.62 84.58) (width 0.2) (layer "F.Cu") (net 18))
 (segment (start 121.62 84.58) (end 122.7 83.5) (width 0.2) (layer "F.Cu") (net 18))
 (segment (start 75 103) (end 89.369 88.631) (width 0.2) (layer "B.Cu") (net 9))
 (segment (start 89.369 76.301) (end 90.47 75.2) (width 0.2) (layer "B.Cu") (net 9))
 (segment (start 89.369 88.631) (end 89.369 76.301) (width 0.2) (layer "B.Cu") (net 9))
 (segment (start 123 94) (end 105.17295 94) (width 0.2) (layer "B.Cu") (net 9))
 (segment (start 105.17295 94) (end 89.369 78.19605) (width 0.2) (layer "B.Cu") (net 9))
 (segment (start 89.369 78.19605) (end 89.369 76.301) (width 0.2) (layer "B.Cu") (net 9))
 (segment (start 59 103) (end 59 102.57295) (width 0.2) (layer "B.Cu") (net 12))
 (segment (start 90.35195 71.221) (end 104.609 71.221) (width 0.2) (layer "B.Cu") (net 12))
 (segment (start 104.609 71.221) (end 105.71 70.12) (width 0.2) (layer "B.Cu") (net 12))
 (segment (start 114 78.41) (end 105.71 70.12) (width 0.2) (layer "B.Cu") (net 12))
 (segment (start 59 102.57295) (end 90.35195 71.221) (width 0.2) (layer "B.Cu") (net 12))
 (segment (start 114 90) (end 114 78.41) (width 0.2) (layer "B.Cu") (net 12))
 (segment (start 54.566599 69.937) (end 56.923599 67.58) (width 0.2) (layer "F.Cu") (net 6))
 (segment (start 56.923599 67.58) (end 90.025 67.58) (width 0.2) (layer "F.Cu") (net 6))
 (segment (start 66.596699 79.4671) (end 91.2829 79.4671) (width 0.2) (layer "F.Cu") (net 14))
 (segment (start 127.6011 112.1011) (end 132.73 117.23) (width 0.2) (layer "F.Cu") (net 14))
 (segment (start 124 108.5) (end 142.602 89.898) (width 0.2) (layer "F.Cu") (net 14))
 (segment (start 126.956091 107.3989) (end 127.6011 108.043909) (width 0.2) (layer "F.Cu") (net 14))
 (segment (start 60.02269 68.8359) (end 60.667699 69.480909) (width 0.2) (layer "F.Cu") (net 14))
 (segment (start 124 108.5) (end 125.1011 107.3989) (width 0.2) (layer "F.Cu") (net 14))
 (segment (start 57.066599 69.937) (end 58.167699 68.8359) (width 0.2) (layer "F.Cu") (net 14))
 (segment (start 142.602 89.898) (end 142.602 79.1) (width 0.2) (layer "F.Cu") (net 14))
 (segment (start 60.667699 69.480909) (end 60.667699 73.5381) (width 0.2) (layer "F.Cu") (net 14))
 (segment (start 60.667699 73.5381) (end 65.796599 78.667) (width 0.2) (layer "F.Cu") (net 14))
 (segment (start 139.201 75.699) (end 116.849 75.699) (width 0.2) (layer "F.Cu") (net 14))
 (segment (start 125.1011 107.3989) (end 126.956091 107.3989) (width 0.2) (layer "F.Cu") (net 14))
 (segment (start 142.602 79.1) (end 139.201 75.699) (width 0.2) (layer "F.Cu") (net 14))
 (segment (start 116.849 75.699) (end 106.19 65.04) (width 0.2) (layer "F.Cu") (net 14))
 (segment (start 65.796599 78.667) (end 66.596699 79.4671) (width 0.2) (layer "F.Cu") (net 14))
 (segment (start 127.6011 108.043909) (end 127.6011 112.1011) (width 0.2) (layer "F.Cu") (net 14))
 (segment (start 58.167699 68.8359) (end 60.02269 68.8359) (width 0.2) (layer "F.Cu") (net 14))
 (segment (start 91.2829 79.4671) (end 105.71 65.04) (width 0.2) (layer "F.Cu") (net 14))
 (segment (start 67 96.13) (end 90.47 72.66) (width 0.2) (layer "B.Cu") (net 8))
 (segment (start 67 100) (end 67 96.13) (width 0.2) (layer "B.Cu") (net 8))
 (segment (start 106.64716 73.761) (end 91.571 73.761) (width 0.2) (layer "B.Cu") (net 8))
 (segment (start 111 87) (end 112.101 85.899) (width 0.2) (layer "B.Cu") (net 8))
 (segment (start 112.101 85.899) (end 112.101 79.21484) (width 0.2) (layer "B.Cu") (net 8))
 (segment (start 91.571 73.761) (end 90.47 72.66) (width 0.2) (layer "B.Cu") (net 8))
 (segment (start 112.101 79.21484) (end 106.64716 73.761) (width 0.2) (layer "B.Cu") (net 8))
 (segment (start 65.796599 76.167) (end 83.978 76.167) (width 0.2) (layer "F.Cu") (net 7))
 (segment (start 83.978 76.167) (end 90.025 70.12) (width 0.2) (layer "F.Cu") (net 7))
 (segment (start 102 115) (end 103.88616 115) (width 0.2) (layer "B.Cu") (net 3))
 (segment (start 113.61384 91.5) (end 109.899 87.78516) (width 0.2) (layer "B.Cu") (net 3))
 (segment (start 106 80) (end 103.74 77.74) (width 0.2) (layer "B.Cu") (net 3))
 (segment (start 103.88616 115) (end 124.101 94.78516) (width 0.2) (layer "B.Cu") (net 3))
 (segment (start 111 80) (end 106 80) (width 0.2) (layer "B.Cu") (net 3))
 (segment (start 103.74 77.74) (end 90.47 77.74) (width 0.2) (layer "B.Cu") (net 3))
 (segment (start 124.101 93.21484) (end 122.38616 91.5) (width 0.2) (layer "B.Cu") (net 3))
 (segment (start 109.899 81.101) (end 111 80) (width 0.2) (layer "B.Cu") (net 3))
 (segment (start 109.899 87.78516) (end 109.899 81.101) (width 0.2) (layer "B.Cu") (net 3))
 (segment (start 124.101 94.78516) (end 124.101 93.21484) (width 0.2) (layer "B.Cu") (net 3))
 (segment (start 122.38616 91.5) (end 113.61384 91.5) (width 0.2) (layer "B.Cu") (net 3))
 (segment (start 137.4 86.5) (end 140.002 86.5) (width 0.2) (layer "F.Cu") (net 1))
 (segment (start 139.3 72.5) (end 146.3 79.5) (width 0.2) (layer "F.Cu") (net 1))
 (segment (start 142.201 81.201) (end 140.5 79.5) (width 0.2) (layer "F.Cu") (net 1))
 (segment (start 137.4 72.5) (end 139.3 72.5) (width 0.2) (layer "F.Cu") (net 1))
 (segment (start 142.201 84.301) (end 142.201 81.201) (width 0.2) (layer "F.Cu") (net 1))
 (segment (start 121.099 81.101) (end 109.071 81.101) (width 0.2) (layer "F.Cu") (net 1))
 (segment (start 109.071 81.101) (end 105.71 77.74) (width 0.2) (layer "F.Cu") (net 1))
 (segment (start 128.5 79.5) (end 140.5 79.5) (width 0.2) (layer "F.Cu") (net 1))
 (segment (start 140.002 86.5) (end 142.201 84.301) (width 0.2) (layer "F.Cu") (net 1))
 (segment (start 122.7 79.5) (end 121.099 81.101) (width 0.2) (layer "F.Cu") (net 1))
 (segment (start 59.566599 74.937) (end 65.796599 81.167) (width 0.2) (layer "F.Cu") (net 13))
 (segment (start 126.5 108.5) (end 126.5 113.5) (width 0.2) (layer "F.Cu") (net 13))
 (segment (start 75.203 110.801) (end 70.199 110.801) (width 0.2) (layer "F.Cu") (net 13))
 (segment (start 125.3989 109.6011) (end 90.7009 109.6011) (width 0.2) (layer "F.Cu") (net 13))
 (segment (start 79.099 117.801) (end 79.099 114.697) (width 0.2) (layer "F.Cu") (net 13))
 (segment (start 70.199 110.801) (end 69.798 110.4) (width 0.2) (layer "F.Cu") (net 13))
 (segment (start 69.798 85.168401) (end 65.796599 81.167) (width 0.2) (layer "F.Cu") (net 13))
 (segment (start 59.566599 69.937) (end 59.566599 74.937) (width 0.2) (layer "F.Cu") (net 13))
 (segment (start 126.5 113.5) (end 132.73 119.73) (width 0.2) (layer "F.Cu") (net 13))
 (segment (start 90.7009 109.6011) (end 82.501 117.801) (width 0.2) (layer "F.Cu") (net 13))
 (segment (start 69.798 110.4) (end 69.798 85.168401) (width 0.2) (layer "F.Cu") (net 13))
 (segment (start 82.501 117.801) (end 79.099 117.801) (width 0.2) (layer "F.Cu") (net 13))
 (segment (start 126.5 108.5) (end 125.3989 109.6011) (width 0.2) (layer "F.Cu") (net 13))
 (segment (start 79.099 114.697) (end 75.203 110.801) (width 0.2) (layer "F.Cu") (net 13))
 (segment (start 88.601599 85.168401) (end 106.19 67.58) (width 0.2) (layer "F.Cu") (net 13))
 (segment (start 69.798 85.168401) (end 88.601599 85.168401) (width 0.2) (layer "F.Cu") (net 13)))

